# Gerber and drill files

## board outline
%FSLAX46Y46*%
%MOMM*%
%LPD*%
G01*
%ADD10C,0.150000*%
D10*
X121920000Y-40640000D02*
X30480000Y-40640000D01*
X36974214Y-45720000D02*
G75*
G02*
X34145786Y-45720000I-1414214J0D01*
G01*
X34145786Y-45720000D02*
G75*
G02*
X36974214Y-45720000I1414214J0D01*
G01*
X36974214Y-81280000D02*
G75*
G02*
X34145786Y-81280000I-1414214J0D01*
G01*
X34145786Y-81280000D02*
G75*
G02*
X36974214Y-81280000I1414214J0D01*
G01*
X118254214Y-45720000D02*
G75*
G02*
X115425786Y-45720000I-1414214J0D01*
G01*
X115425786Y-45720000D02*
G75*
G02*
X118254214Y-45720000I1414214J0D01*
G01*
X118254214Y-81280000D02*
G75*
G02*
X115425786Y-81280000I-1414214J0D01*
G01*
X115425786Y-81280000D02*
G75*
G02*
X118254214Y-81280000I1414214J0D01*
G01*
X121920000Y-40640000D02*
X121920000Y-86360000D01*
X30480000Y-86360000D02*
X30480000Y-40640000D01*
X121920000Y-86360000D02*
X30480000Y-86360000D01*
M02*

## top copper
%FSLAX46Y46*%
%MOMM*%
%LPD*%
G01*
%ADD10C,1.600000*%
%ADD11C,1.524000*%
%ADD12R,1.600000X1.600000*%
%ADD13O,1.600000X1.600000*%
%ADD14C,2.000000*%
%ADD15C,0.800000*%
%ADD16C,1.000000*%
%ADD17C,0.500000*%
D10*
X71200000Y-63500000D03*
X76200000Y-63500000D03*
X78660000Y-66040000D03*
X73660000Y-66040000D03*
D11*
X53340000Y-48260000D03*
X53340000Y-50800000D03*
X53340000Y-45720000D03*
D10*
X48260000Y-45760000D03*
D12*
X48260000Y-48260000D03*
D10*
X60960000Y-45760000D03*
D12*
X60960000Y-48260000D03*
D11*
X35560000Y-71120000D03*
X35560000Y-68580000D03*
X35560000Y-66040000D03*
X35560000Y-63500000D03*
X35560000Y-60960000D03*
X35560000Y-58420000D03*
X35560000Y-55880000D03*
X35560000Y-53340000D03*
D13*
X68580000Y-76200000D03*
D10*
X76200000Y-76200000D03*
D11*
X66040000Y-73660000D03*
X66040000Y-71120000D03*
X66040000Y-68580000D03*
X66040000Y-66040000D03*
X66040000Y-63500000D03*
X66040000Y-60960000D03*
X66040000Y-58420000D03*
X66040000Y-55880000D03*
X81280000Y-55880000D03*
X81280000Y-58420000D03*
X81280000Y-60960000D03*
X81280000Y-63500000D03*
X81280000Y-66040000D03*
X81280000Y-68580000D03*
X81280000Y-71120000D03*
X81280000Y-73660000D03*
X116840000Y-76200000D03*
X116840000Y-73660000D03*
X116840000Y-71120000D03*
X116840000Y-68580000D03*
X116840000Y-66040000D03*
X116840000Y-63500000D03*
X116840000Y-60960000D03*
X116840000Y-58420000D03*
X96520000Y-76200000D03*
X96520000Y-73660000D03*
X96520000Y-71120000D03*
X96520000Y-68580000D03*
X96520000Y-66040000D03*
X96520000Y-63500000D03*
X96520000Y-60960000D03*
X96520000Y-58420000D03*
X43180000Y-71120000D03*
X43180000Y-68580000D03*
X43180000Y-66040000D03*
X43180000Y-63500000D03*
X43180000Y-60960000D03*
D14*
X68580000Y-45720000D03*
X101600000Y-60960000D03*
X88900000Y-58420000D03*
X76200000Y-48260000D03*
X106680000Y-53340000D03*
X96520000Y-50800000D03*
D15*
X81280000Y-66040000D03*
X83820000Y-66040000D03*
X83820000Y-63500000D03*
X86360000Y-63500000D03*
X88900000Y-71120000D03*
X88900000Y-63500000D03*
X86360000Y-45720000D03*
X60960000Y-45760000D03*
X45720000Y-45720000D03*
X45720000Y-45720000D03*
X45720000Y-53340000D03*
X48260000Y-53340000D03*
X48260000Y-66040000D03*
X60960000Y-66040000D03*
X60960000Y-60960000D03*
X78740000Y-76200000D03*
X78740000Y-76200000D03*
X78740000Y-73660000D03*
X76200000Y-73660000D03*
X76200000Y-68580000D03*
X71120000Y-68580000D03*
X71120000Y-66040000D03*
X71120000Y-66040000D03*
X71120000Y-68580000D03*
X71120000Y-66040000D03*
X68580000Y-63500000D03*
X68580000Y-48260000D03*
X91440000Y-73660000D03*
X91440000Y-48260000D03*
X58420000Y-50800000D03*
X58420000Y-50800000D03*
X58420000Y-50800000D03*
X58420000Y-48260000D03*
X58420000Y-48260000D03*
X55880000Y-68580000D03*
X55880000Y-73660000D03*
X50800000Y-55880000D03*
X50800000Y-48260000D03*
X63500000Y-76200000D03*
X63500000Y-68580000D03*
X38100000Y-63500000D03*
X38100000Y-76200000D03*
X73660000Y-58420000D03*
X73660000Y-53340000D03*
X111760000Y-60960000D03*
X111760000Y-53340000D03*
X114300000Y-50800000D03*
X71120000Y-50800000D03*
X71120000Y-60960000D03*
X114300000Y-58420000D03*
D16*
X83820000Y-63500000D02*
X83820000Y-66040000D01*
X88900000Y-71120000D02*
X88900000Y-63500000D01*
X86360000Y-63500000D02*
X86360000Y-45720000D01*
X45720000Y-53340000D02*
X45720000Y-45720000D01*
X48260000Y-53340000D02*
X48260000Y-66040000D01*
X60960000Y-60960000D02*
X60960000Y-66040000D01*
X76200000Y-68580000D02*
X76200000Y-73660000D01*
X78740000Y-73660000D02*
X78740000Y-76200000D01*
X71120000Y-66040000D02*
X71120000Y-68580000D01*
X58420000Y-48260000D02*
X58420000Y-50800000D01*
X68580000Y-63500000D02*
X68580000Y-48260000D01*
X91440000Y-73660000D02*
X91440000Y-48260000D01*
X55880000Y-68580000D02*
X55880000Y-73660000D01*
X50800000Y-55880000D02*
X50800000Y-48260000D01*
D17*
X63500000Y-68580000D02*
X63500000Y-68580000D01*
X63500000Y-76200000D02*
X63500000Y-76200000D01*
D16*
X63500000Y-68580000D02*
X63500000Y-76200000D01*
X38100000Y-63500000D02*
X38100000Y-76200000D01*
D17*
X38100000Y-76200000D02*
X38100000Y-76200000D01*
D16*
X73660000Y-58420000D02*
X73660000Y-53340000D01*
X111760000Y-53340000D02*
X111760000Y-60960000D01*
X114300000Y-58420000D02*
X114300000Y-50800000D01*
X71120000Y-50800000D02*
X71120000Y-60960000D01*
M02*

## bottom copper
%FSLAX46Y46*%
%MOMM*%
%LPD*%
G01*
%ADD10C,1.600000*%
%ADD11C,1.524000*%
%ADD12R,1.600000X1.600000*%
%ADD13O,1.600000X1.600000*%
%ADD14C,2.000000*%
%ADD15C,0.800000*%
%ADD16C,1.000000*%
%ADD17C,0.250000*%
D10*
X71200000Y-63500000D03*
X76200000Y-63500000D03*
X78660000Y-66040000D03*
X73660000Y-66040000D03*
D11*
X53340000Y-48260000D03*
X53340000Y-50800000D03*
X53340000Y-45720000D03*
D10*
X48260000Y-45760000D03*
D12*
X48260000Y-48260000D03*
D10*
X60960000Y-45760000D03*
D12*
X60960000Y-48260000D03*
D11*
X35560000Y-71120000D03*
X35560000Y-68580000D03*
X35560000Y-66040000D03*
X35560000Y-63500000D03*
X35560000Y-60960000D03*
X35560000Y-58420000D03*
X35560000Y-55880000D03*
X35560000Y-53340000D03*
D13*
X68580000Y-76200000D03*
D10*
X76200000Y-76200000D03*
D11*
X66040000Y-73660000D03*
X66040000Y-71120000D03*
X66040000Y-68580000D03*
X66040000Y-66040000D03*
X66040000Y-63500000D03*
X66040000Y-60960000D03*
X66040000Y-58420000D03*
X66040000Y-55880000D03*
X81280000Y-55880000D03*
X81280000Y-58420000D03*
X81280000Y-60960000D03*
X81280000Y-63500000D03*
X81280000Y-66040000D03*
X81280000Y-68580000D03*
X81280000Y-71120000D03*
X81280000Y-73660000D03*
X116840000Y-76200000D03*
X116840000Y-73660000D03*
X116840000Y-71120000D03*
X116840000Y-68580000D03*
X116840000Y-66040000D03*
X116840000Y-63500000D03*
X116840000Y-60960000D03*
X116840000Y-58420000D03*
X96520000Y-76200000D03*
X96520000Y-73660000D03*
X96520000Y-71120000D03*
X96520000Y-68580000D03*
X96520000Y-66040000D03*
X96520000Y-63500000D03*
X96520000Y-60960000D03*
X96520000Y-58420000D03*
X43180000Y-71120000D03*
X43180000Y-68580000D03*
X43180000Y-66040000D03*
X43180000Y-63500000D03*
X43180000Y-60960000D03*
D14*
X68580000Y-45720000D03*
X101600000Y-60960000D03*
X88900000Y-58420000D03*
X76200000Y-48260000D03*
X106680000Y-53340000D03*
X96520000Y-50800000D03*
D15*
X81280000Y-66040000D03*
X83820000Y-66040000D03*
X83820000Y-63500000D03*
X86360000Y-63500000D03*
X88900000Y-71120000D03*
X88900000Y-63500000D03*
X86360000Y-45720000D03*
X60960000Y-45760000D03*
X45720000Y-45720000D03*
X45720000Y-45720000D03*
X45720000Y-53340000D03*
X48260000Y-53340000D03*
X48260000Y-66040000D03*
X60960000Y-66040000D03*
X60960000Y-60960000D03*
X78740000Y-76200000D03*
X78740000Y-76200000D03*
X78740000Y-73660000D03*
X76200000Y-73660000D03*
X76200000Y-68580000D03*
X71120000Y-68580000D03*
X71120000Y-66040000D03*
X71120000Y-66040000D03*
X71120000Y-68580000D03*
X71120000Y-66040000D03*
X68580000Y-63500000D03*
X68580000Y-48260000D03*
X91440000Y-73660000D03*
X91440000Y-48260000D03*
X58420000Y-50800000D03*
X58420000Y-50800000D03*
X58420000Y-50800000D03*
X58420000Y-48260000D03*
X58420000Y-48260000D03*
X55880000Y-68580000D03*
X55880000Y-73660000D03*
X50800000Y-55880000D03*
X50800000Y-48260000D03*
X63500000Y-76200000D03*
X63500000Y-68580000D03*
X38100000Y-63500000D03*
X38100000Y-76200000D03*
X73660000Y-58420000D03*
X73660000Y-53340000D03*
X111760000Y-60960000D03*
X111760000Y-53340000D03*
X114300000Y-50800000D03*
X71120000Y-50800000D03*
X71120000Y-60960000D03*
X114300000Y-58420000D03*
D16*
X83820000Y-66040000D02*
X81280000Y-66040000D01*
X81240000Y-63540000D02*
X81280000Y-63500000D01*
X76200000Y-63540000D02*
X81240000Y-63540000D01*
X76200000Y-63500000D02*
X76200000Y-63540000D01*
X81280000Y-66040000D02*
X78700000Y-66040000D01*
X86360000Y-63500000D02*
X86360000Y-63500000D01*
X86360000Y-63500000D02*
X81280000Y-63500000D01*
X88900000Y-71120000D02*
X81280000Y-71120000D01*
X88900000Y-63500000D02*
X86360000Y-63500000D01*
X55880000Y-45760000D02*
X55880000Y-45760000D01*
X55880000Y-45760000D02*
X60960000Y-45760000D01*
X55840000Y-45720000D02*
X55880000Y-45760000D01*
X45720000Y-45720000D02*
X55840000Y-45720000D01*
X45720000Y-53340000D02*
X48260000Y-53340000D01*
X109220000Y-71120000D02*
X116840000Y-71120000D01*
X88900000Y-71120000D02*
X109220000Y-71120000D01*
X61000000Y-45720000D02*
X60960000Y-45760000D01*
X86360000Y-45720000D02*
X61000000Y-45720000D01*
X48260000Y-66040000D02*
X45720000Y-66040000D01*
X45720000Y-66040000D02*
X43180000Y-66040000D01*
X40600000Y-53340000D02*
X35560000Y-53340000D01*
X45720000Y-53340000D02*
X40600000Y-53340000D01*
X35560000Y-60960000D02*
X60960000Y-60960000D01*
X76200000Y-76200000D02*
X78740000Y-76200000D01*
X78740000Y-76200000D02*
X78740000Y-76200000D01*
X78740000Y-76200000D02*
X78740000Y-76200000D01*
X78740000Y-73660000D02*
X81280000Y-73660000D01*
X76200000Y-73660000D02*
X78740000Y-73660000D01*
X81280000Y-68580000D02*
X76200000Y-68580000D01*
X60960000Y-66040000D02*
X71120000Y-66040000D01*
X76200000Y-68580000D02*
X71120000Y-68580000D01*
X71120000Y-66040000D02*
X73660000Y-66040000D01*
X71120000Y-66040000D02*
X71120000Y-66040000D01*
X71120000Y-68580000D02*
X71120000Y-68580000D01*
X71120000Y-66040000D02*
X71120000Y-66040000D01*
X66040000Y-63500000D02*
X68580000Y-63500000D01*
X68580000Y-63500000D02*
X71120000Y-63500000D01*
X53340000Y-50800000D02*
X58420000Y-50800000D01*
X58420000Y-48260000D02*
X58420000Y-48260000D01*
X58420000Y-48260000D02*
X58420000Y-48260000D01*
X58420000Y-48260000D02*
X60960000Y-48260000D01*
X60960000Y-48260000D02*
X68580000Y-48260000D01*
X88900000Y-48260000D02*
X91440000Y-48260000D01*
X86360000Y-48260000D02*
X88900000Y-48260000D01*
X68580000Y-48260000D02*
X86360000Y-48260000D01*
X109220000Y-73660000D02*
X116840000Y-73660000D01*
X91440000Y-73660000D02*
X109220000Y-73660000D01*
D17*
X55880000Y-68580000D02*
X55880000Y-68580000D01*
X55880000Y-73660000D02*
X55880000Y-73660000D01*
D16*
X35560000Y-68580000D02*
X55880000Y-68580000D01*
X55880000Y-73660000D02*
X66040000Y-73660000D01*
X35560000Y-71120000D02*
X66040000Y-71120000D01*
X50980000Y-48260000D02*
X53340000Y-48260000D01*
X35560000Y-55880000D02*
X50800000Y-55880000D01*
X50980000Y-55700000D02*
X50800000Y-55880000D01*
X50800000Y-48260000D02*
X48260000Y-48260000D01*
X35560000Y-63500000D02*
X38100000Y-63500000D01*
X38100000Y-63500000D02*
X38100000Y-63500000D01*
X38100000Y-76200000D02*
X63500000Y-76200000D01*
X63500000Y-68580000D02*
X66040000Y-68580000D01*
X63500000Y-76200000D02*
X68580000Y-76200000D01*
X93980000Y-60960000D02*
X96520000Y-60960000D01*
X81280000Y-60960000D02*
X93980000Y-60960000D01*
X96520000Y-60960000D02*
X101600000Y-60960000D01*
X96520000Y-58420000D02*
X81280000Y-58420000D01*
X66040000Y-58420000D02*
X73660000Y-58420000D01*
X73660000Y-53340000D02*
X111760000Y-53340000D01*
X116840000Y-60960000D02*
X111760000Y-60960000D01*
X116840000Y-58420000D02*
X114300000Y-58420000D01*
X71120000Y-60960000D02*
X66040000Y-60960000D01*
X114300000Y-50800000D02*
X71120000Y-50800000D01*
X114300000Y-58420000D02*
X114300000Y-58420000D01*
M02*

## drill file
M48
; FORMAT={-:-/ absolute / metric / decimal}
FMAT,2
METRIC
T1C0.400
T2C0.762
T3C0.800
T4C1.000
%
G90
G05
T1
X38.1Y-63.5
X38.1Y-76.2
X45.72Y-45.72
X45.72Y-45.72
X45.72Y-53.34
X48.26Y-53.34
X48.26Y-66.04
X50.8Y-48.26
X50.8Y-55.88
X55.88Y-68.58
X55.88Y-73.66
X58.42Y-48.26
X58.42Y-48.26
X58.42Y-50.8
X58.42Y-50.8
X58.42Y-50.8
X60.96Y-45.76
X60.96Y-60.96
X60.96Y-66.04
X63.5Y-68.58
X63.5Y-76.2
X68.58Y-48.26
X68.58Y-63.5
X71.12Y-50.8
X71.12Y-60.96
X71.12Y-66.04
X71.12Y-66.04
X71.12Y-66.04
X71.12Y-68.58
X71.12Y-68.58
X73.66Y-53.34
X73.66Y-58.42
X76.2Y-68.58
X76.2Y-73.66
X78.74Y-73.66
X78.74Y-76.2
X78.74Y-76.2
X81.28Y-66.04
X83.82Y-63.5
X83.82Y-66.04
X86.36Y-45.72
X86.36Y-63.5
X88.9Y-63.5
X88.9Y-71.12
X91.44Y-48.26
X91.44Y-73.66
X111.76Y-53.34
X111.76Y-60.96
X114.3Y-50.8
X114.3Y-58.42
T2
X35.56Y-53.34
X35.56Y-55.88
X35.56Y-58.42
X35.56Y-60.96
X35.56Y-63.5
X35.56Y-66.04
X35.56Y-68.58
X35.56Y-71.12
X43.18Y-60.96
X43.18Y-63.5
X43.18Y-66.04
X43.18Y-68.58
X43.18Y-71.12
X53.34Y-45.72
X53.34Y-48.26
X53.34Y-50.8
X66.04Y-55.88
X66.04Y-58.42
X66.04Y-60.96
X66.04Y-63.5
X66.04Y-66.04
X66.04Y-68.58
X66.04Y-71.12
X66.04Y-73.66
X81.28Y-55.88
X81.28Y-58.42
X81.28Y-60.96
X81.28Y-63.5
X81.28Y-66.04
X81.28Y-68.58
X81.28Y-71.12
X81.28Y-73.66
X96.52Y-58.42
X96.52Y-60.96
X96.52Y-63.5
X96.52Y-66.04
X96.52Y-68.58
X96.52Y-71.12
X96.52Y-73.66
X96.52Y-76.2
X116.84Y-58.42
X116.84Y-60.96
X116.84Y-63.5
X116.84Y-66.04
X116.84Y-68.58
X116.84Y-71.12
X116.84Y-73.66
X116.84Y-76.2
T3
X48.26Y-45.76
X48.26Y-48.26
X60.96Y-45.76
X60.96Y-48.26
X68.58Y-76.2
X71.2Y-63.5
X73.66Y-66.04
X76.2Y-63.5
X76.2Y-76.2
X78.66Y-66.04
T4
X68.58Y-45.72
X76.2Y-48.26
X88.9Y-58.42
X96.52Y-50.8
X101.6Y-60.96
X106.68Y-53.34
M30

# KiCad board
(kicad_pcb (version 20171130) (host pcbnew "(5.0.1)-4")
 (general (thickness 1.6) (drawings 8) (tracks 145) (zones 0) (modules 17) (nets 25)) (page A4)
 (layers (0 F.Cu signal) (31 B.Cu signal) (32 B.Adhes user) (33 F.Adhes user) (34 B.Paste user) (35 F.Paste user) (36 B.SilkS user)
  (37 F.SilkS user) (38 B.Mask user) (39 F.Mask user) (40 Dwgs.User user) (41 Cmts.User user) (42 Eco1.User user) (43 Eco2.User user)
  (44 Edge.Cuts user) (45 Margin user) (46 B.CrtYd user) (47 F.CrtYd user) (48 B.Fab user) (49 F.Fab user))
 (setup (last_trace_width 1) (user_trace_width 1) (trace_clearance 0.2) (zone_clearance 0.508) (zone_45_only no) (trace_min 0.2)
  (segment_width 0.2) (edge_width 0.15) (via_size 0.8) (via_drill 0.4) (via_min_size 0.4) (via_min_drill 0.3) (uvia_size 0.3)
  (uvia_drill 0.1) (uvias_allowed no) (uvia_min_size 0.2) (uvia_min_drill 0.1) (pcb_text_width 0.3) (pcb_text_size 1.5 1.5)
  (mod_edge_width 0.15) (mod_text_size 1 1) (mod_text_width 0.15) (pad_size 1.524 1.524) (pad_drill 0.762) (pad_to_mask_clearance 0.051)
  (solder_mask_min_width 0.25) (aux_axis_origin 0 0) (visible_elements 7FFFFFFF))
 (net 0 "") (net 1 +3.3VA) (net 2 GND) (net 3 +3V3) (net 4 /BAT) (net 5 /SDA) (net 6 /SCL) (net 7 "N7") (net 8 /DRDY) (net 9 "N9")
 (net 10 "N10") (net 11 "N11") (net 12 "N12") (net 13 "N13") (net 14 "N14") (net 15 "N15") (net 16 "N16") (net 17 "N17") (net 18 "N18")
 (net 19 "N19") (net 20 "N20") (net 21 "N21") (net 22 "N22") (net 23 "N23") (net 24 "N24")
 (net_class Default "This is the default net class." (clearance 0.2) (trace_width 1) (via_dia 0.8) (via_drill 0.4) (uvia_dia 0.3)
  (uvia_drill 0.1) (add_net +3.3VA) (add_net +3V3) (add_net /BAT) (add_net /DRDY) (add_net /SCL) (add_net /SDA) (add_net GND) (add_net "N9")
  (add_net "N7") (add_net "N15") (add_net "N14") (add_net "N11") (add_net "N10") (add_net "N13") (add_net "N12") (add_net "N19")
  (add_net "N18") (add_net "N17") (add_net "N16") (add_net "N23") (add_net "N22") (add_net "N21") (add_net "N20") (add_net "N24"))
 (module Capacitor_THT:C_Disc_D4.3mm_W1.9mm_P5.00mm (layer F.Cu) (at 76.2 63.5 180)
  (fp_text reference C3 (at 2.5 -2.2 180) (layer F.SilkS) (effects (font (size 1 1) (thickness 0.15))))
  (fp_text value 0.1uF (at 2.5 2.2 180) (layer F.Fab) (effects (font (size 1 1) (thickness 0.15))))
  (pad 2 thru_hole circle (at 5 0 180) (size 1.6 1.6) (drill 0.8) (layers *.Cu *.Mask) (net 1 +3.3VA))
  (pad 1 thru_hole circle (at 0 0 180) (size 1.6 1.6) (drill 0.8) (layers *.Cu *.Mask) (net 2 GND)))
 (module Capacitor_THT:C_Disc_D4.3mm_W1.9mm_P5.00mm (layer F.Cu) (at 73.66 66.04)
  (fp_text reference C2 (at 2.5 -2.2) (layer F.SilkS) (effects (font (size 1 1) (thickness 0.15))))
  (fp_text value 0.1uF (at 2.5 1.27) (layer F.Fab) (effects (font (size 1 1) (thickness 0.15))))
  (pad 2 thru_hole circle (at 5 0) (size 1.6 1.6) (drill 0.8) (layers *.Cu *.Mask) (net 2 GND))
  (pad 1 thru_hole circle (at 0 0) (size 1.6 1.6) (drill 0.8) (layers *.Cu *.Mask) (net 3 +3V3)))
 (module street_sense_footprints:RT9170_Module (layer F.Cu) (at 55.88 48.26 270)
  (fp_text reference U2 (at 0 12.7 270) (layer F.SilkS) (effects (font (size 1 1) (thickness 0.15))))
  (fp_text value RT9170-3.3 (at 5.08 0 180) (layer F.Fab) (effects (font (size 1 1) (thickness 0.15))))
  (pad 3 thru_hole circle (at 0 2.54 270) (size 1.524 1.524) (drill 0.762) (layers *.Cu *.Mask) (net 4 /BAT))
  (pad 2 thru_hole circle (at 2.54 2.54 270) (size 1.524 1.524) (drill 0.762) (layers *.Cu *.Mask) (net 1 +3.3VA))
  (pad 1 thru_hole circle (at -2.54 2.54 270) (size 1.524 1.524) (drill 0.762) (layers *.Cu *.Mask) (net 2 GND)))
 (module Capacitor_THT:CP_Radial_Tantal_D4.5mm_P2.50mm (layer F.Cu) (at 48.26 48.26 90)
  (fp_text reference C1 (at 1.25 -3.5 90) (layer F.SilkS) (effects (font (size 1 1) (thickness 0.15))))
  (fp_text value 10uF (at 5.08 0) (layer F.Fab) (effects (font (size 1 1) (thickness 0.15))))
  (pad 2 thru_hole circle (at 2.5 0 90) (size 1.6 1.6) (drill 0.8) (layers *.Cu *.Mask) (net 2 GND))
  (pad 1 thru_hole rect (at 0 0 90) (size 1.6 1.6) (drill 0.8) (layers *.Cu *.Mask) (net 4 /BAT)))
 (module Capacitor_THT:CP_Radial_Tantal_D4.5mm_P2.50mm (layer F.Cu) (at 60.96 48.26 90)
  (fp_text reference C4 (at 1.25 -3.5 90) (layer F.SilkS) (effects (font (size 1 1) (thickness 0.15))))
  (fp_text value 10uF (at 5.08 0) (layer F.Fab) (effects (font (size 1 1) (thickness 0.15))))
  (pad 2 thru_hole circle (at 2.5 0 90) (size 1.6 1.6) (drill 0.8) (layers *.Cu *.Mask) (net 2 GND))
  (pad 1 thru_hole rect (at 0 0 90) (size 1.6 1.6) (drill 0.8) (layers *.Cu *.Mask) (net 1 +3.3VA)))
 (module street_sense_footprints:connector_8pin (layer F.Cu) (at 35.56 50.8)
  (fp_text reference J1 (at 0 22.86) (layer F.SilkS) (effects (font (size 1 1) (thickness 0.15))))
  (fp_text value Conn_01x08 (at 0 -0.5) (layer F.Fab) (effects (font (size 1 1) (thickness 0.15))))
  (pad 8 thru_hole circle (at 0 20.32) (size 1.524 1.524) (drill 0.762) (layers *.Cu *.Mask) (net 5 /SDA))
  (pad 7 thru_hole circle (at 0 17.78) (size 1.524 1.524) (drill 0.762) (layers *.Cu *.Mask) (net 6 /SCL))
  (pad 6 thru_hole circle (at 0 15.24) (size 1.524 1.524) (drill 0.762) (layers *.Cu *.Mask) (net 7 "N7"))
  (pad 5 thru_hole circle (at 0 12.7) (size 1.524 1.524) (drill 0.762) (layers *.Cu *.Mask) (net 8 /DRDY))
  (pad 4 thru_hole circle (at 0 10.16) (size 1.524 1.524) (drill 0.762) (layers *.Cu *.Mask) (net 3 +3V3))
  (pad 3 thru_hole circle (at 0 7.62) (size 1.524 1.524) (drill 0.762) (layers *.Cu *.Mask) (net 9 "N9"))
  (pad 2 thru_hole circle (at 0 5.08) (size 1.524 1.524) (drill 0.762) (layers *.Cu *.Mask) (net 4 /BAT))
  (pad 1 thru_hole circle (at 0 2.54) (size 1.524 1.524) (drill 0.762) (layers *.Cu *.Mask) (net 2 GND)))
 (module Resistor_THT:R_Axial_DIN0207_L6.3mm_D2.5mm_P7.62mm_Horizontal (layer F.Cu) (at 76.2 76.2 180)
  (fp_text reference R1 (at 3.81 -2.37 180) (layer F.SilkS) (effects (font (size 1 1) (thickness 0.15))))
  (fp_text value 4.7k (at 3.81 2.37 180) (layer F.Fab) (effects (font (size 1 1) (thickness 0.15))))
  (pad 2 thru_hole oval (at 7.62 0 180) (size 1.6 1.6) (drill 0.8) (layers *.Cu *.Mask) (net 8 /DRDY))
  (pad 1 thru_hole circle (at 0 0 180) (size 1.6 1.6) (drill 0.8) (layers *.Cu *.Mask) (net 3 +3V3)))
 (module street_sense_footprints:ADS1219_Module (layer F.Cu) (at 76.2 76.2 180)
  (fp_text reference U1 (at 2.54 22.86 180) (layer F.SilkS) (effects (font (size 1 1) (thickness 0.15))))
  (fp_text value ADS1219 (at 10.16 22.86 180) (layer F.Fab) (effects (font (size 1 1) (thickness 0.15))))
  (pad 16 thru_hole circle (at 10.16 2.54 180) (size 1.524 1.524) (drill 0.762) (layers *.Cu *.Mask) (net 6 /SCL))
  (pad 15 thru_hole circle (at 10.16 5.08 180) (size 1.524 1.524) (drill 0.762) (layers *.Cu *.Mask) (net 5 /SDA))
  (pad 14 thru_hole circle (at 10.16 7.62 180) (size 1.524 1.524) (drill 0.762) (layers *.Cu *.Mask) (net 8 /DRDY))
  (pad 13 thru_hole circle (at 10.16 10.16 180) (size 1.524 1.524) (drill 0.762) (layers *.Cu *.Mask) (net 3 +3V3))
  (pad 12 thru_hole circle (at 10.16 12.7 180) (size 1.524 1.524) (drill 0.762) (layers *.Cu *.Mask) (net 1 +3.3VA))
  (pad 11 thru_hole circle (at 10.16 15.24 180) (size 1.524 1.524) (drill 0.762) (layers *.Cu *.Mask) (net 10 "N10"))
  (pad 10 thru_hole circle (at 10.16 17.78 180) (size 1.524 1.524) (drill 0.762) (layers *.Cu *.Mask) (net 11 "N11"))
  (pad 9 thru_hole circle (at 10.16 20.32 180) (size 1.524 1.524) (drill 0.762) (layers *.Cu *.Mask) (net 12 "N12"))
  (pad 8 thru_hole circle (at -5.08 20.32 180) (size 1.524 1.524) (drill 0.762) (layers *.Cu *.Mask) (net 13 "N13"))
  (pad 7 thru_hole circle (at -5.08 17.78 180) (size 1.524 1.524) (drill 0.762) (layers *.Cu *.Mask) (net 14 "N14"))
  (pad 6 thru_hole circle (at -5.08 15.24 180) (size 1.524 1.524) (drill 0.762) (layers *.Cu *.Mask) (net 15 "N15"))
  (pad 5 thru_hole circle (at -5.08 12.7 180) (size 1.524 1.524) (drill 0.762) (layers *.Cu *.Mask) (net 2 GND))
  (pad 4 thru_hole circle (at -5.08 10.16 180) (size 1.524 1.524) (drill 0.762) (layers *.Cu *.Mask) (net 2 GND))
  (pad 3 thru_hole circle (at -5.08 7.62 180) (size 1.524 1.524) (drill 0.762) (layers *.Cu *.Mask) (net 3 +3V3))
  (pad 2 thru_hole circle (at -5.08 5.08 180) (size 1.524 1.524) (drill 0.762) (layers *.Cu *.Mask) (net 2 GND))
  (pad 1 thru_hole circle (at -5.08 2.54 180) (size 1.524 1.524) (drill 0.762) (layers *.Cu *.Mask) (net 3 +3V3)))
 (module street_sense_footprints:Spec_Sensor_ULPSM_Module (layer F.Cu) (at 119.38 68.58 270)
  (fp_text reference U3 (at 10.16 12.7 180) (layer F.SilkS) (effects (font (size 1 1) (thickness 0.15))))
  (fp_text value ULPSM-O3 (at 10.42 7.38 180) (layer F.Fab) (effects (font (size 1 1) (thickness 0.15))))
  (pad 8 thru_hole circle (at 7.62 2.54 270) (size 1.524 1.524) (drill 0.762) (layers *.Cu *.Mask) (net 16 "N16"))
  (pad 7 thru_hole circle (at 5.08 2.54 270) (size 1.524 1.524) (drill 0.762) (layers *.Cu *.Mask) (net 1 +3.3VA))
  (pad 6 thru_hole circle (at 2.54 2.54 270) (size 1.524 1.524) (drill 0.762) (layers *.Cu *.Mask) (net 2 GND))
  (pad 5 thru_hole circle (at 0 2.54 270) (size 1.524 1.524) (drill 0.762) (layers *.Cu *.Mask) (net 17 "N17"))
  (pad 4 thru_hole circle (at -2.54 2.54 270) (size 1.524 1.524) (drill 0.762) (layers *.Cu *.Mask) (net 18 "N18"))
  (pad 3 thru_hole circle (at -5.08 2.54 270) (size 1.524 1.524) (drill 0.762) (layers *.Cu *.Mask) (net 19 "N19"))
  (pad 2 thru_hole circle (at -7.62 2.54 270) (size 1.524 1.524) (drill 0.762) (layers *.Cu *.Mask) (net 11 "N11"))
  (pad 1 thru_hole circle (at -10.16 2.54 270) (size 1.524 1.524) (drill 0.762) (layers *.Cu *.Mask) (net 10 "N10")))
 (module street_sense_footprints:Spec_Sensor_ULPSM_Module (layer F.Cu) (at 99.06 68.58 270)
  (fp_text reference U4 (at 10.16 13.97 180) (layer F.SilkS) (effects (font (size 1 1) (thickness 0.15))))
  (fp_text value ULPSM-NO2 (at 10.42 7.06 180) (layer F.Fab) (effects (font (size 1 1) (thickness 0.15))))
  (pad 8 thru_hole circle (at 7.62 2.54 270) (size 1.524 1.524) (drill 0.762) (layers *.Cu *.Mask) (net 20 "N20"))
  (pad 7 thru_hole circle (at 5.08 2.54 270) (size 1.524 1.524) (drill 0.762) (layers *.Cu *.Mask) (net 1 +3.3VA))
  (pad 6 thru_hole circle (at 2.54 2.54 270) (size 1.524 1.524) (drill 0.762) (layers *.Cu *.Mask) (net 2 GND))
  (pad 5 thru_hole circle (at 0 2.54 270) (size 1.524 1.524) (drill 0.762) (layers *.Cu *.Mask) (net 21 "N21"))
  (pad 4 thru_hole circle (at -2.54 2.54 270) (size 1.524 1.524) (drill 0.762) (layers *.Cu *.Mask) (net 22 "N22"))
  (pad 3 thru_hole circle (at -5.08 2.54 270) (size 1.524 1.524) (drill 0.762) (layers *.Cu *.Mask) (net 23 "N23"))
  (pad 2 thru_hole circle (at -7.62 2.54 270) (size 1.524 1.524) (drill 0.762) (layers *.Cu *.Mask) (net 15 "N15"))
  (pad 1 thru_hole circle (at -10.16 2.54 270) (size 1.524 1.524) (drill 0.762) (layers *.Cu *.Mask) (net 14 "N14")))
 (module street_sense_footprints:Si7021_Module (layer F.Cu) (at 53.34 66.04 270)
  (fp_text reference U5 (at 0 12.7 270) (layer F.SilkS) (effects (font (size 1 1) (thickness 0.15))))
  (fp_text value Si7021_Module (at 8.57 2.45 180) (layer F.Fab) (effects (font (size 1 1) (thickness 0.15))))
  (pad 5 thru_hole circle (at 5.08 10.16 270) (size 1.524 1.524) (drill 0.762) (layers *.Cu *.Mask) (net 5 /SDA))
  (pad 4 thru_hole circle (at 2.54 10.16 270) (size 1.524 1.524) (drill 0.762) (layers *.Cu *.Mask) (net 6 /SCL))
  (pad 3 thru_hole circle (at 0 10.16 270) (size 1.524 1.524) (drill 0.762) (layers *.Cu *.Mask) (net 2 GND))
  (pad 2 thru_hole circle (at -2.54 10.16 270) (size 1.524 1.524) (drill 0.762) (layers *.Cu *.Mask) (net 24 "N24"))
  (pad 1 thru_hole circle (at -5.08 10.16 270) (size 1.524 1.524) (drill 0.762) (layers *.Cu *.Mask) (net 3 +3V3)))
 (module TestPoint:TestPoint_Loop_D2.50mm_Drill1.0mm (layer F.Cu) (at 68.58 45.72)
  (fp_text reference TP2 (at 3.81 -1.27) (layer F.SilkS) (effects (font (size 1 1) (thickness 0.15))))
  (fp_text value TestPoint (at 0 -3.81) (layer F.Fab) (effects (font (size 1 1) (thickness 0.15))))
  (pad 1 thru_hole circle (at 0 0) (size 2 2) (drill 1) (layers *.Cu *.Mask) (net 2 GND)))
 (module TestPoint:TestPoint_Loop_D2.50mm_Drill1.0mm (layer F.Cu) (at 101.6 60.96)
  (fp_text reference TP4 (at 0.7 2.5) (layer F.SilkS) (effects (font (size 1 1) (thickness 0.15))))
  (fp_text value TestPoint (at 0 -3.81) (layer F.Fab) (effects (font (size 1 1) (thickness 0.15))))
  (pad 1 thru_hole circle (at 0 0) (size 2 2) (drill 1) (layers *.Cu *.Mask) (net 15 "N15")))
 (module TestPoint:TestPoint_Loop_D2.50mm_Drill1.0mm (layer F.Cu) (at 88.9 58.42)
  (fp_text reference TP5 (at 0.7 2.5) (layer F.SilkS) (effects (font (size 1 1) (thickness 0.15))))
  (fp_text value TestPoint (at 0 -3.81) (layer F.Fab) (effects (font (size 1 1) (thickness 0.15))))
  (pad 1 thru_hole circle (at 0 0) (size 2 2) (drill 1) (layers *.Cu *.Mask) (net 14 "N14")))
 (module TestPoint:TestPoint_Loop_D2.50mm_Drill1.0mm (layer F.Cu) (at 76.2 48.26)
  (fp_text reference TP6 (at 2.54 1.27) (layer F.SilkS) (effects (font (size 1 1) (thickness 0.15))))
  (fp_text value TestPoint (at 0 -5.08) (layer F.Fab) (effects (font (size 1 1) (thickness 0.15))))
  (pad 1 thru_hole circle (at 0 0) (size 2 2) (drill 1) (layers *.Cu *.Mask) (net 1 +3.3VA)))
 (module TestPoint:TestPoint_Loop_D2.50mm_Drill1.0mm (layer F.Cu) (at 106.68 53.34)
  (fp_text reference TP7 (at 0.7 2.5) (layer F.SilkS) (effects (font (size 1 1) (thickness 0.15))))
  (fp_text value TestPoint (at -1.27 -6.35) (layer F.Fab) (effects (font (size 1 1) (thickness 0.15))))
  (pad 1 thru_hole circle (at 0 0) (size 2 2) (drill 1) (layers *.Cu *.Mask) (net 11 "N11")))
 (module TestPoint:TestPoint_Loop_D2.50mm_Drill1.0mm (layer F.Cu) (at 96.52 50.8)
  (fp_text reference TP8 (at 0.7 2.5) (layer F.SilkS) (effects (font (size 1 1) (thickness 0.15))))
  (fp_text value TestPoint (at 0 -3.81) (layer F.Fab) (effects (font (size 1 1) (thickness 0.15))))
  (pad 1 thru_hole circle (at 0 0) (size 2 2) (drill 1) (layers *.Cu *.Mask) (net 10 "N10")))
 (gr_line (start 121.92 40.64) (end 30.48 40.64) (layer Edge.Cuts) (width 0.15))
 (gr_circle (center 35.56 45.72) (end 36.974214 45.72) (layer Edge.Cuts) (width 0.15))
 (gr_circle (center 35.56 81.28) (end 36.974214 81.28) (layer Edge.Cuts) (width 0.15))
 (gr_circle (center 116.84 45.72) (end 115.84 46.72) (layer Edge.Cuts) (width 0.15))
 (gr_circle (center 116.84 81.28) (end 118.254214 81.28) (layer Edge.Cuts) (width 0.15))
 (gr_line (start 121.92 40.64) (end 121.92 86.36) (layer Edge.Cuts) (width 0.15))
 (gr_line (start 30.48 86.36) (end 30.48 40.64) (layer Edge.Cuts) (width 0.15))
 (gr_line (start 121.92 86.36) (end 30.48 86.36) (layer Edge.Cuts) (width 0.15))
 (via (at 81.28 66.04) (size 0.8) (drill 0.4) (layers F.Cu B.Cu) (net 2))
 (via (at 83.82 66.04) (size 0.8) (drill 0.4) (layers F.Cu B.Cu) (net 2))
 (segment (start 83.82 66.04) (end 81.28 66.04) (width 1) (layer B.Cu) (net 2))
 (segment (start 81.24 63.54) (end 81.28 63.5) (width 1) (layer B.Cu) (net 2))
 (segment (start 76.2 63.54) (end 81.24 63.54) (width 1) (layer B.Cu) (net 2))
 (segment (start 76.2 63.5) (end 76.2 63.54) (width 1) (layer B.Cu) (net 2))
 (segment (start 83.82 63.5) (end 83.82 66.04) (width 1) (layer F.Cu) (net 2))
 (via (at 83.82 63.5) (size 0.8) (drill 0.4) (layers F.Cu B.Cu) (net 2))
 (segment (start 81.28 66.04) (end 78.7 66.04) (width 1) (layer B.Cu) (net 2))
 (segment (start 86.36 63.5) (end 86.36 63.5) (width 1) (layer B.Cu) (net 2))
 (segment (start 86.36 63.5) (end 81.28 63.5) (width 1) (layer B.Cu) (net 2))
 (via (at 86.36 63.5) (size 0.8) (drill 0.4) (layers F.Cu B.Cu) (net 2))
 (via (at 88.9 71.12) (size 0.8) (drill 0.4) (layers F.Cu B.Cu) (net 2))
 (segment (start 88.9 71.12) (end 81.28 71.12) (width 1) (layer B.Cu) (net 2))
 (via (at 88.9 63.5) (size 0.8) (drill 0.4) (layers F.Cu B.Cu) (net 2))
 (segment (start 88.9 71.12) (end 88.9 63.5) (width 1) (layer F.Cu) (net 2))
 (segment (start 88.9 63.5) (end 86.36 63.5) (width 1) (layer B.Cu) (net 2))
 (via (at 86.36 45.72) (size 0.8) (drill 0.4) (layers F.Cu B.Cu) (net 2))
 (segment (start 55.88 45.76) (end 55.88 45.76) (width 1) (layer B.Cu) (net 2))
 (via (at 60.96 45.76) (size 0.8) (drill 0.4) (layers F.Cu B.Cu) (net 2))
 (segment (start 55.88 45.76) (end 60.96 45.76) (width 1) (layer B.Cu) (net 2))
 (segment (start 86.36 63.5) (end 86.36 45.72) (width 1) (layer F.Cu) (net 2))
 (segment (start 45.72 53.34) (end 45.72 45.72) (width 1) (layer F.Cu) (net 2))
 (segment (start 55.84 45.72) (end 55.88 45.76) (width 1) (layer B.Cu) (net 2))
 (segment (start 45.72 45.72) (end 55.84 45.72) (width 1) (layer B.Cu) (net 2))
 (via (at 45.72 45.72) (size 0.8) (drill 0.4) (layers F.Cu B.Cu) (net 2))
 (via (at 45.72 45.72) (size 0.8) (drill 0.4) (layers F.Cu B.Cu) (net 2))
 (via (at 45.72 53.34) (size 0.8) (drill 0.4) (layers F.Cu B.Cu) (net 2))
 (segment (start 45.72 53.34) (end 48.26 53.34) (width 1) (layer B.Cu) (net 2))
 (via (at 48.26 53.34) (size 0.8) (drill 0.4) (layers F.Cu B.Cu) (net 2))
 (segment (start 109.22 71.12) (end 116.84 71.12) (width 1) (layer B.Cu) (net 2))
 (segment (start 88.9 71.12) (end 109.22 71.12) (width 1) (layer B.Cu) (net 2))
 (segment (start 61 45.72) (end 60.96 45.76) (width 1) (layer B.Cu) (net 2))
 (segment (start 86.36 45.72) (end 61 45.72) (width 1) (layer B.Cu) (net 2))
 (segment (start 48.26 53.34) (end 48.26 66.04) (width 1) (layer F.Cu) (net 2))
 (segment (start 48.26 66.04) (end 45.72 66.04) (width 1) (layer B.Cu) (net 2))
 (segment (start 45.72 66.04) (end 43.18 66.04) (width 1) (layer B.Cu) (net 2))
 (via (at 48.26 66.04) (size 0.8) (drill 0.4) (layers F.Cu B.Cu) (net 2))
 (segment (start 40.6 53.34) (end 35.56 53.34) (width 1) (layer B.Cu) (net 2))
 (segment (start 45.72 53.34) (end 40.6 53.34) (width 1) (layer B.Cu) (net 2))
 (via (at 60.96 66.04) (size 0.8) (drill 0.4) (layers F.Cu B.Cu) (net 3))
 (segment (start 35.56 60.96) (end 60.96 60.96) (width 1) (layer B.Cu) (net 3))
 (segment (start 60.96 60.96) (end 60.96 66.04) (width 1) (layer F.Cu) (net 3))
 (via (at 60.96 60.96) (size 0.8) (drill 0.4) (layers F.Cu B.Cu) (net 3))
 (segment (start 76.2 68.58) (end 76.2 73.66) (width 1) (layer F.Cu) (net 3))
 (segment (start 76.2 76.2) (end 78.74 76.2) (width 1) (layer B.Cu) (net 3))
 (segment (start 78.74 76.2) (end 78.74 76.2) (width 1) (layer B.Cu) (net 3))
 (via (at 78.74 76.2) (size 0.8) (drill 0.4) (layers F.Cu B.Cu) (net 3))
 (segment (start 78.74 76.2) (end 78.74 76.2) (width 1) (layer B.Cu) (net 3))
 (via (at 78.74 76.2) (size 0.8) (drill 0.4) (layers F.Cu B.Cu) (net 3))
 (segment (start 78.74 73.66) (end 81.28 73.66) (width 1) (layer B.Cu) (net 3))
 (via (at 78.74 73.66) (size 0.8) (drill 0.4) (layers F.Cu B.Cu) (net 3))
 (segment (start 78.74 73.66) (end 78.74 76.2) (width 1) (layer F.Cu) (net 3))
 (segment (start 76.2 73.66) (end 78.74 73.66) (width 1) (layer B.Cu) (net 3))
 (via (at 76.2 73.66) (size 0.8) (drill 0.4) (layers F.Cu B.Cu) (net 3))
 (via (at 76.2 68.58) (size 0.8) (drill 0.4) (layers F.Cu B.Cu) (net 3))
 (segment (start 81.28 68.58) (end 76.2 68.58) (width 1) (layer B.Cu) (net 3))
 (segment (start 60.96 66.04) (end 71.12 66.04) (width 1) (layer B.Cu) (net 3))
 (segment (start 76.2 68.58) (end 71.12 68.58) (width 1) (layer B.Cu) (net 3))
 (via (at 71.12 68.58) (size 0.8) (drill 0.4) (layers F.Cu B.Cu) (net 3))
 (segment (start 71.12 66.04) (end 73.66 66.04) (width 1) (layer B.Cu) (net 3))
 (via (at 71.12 66.04) (size 0.8) (drill 0.4) (layers F.Cu B.Cu) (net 3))
 (segment (start 71.12 66.04) (end 71.12 66.04) (width 1) (layer B.Cu) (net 3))
 (via (at 71.12 66.04) (size 0.8) (drill 0.4) (layers F.Cu B.Cu) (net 3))
 (segment (start 71.12 68.58) (end 71.12 68.58) (width 1) (layer B.Cu) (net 3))
 (via (at 71.12 68.58) (size 0.8) (drill 0.4) (layers F.Cu B.Cu) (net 3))
 (segment (start 71.12 66.04) (end 71.12 66.04) (width 1) (layer B.Cu) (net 3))
 (via (at 71.12 66.04) (size 0.8) (drill 0.4) (layers F.Cu B.Cu) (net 3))
 (segment (start 71.12 66.04) (end 71.12 68.58) (width 1) (layer F.Cu) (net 3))
 (via (at 68.58 63.5) (size 0.8) (drill 0.4) (layers F.Cu B.Cu) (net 1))
 (segment (start 66.04 63.5) (end 68.58 63.5) (width 1) (layer B.Cu) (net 1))
 (via (at 68.58 48.26) (size 0.8) (drill 0.4) (layers F.Cu B.Cu) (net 1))
 (via (at 91.44 73.66) (size 0.8) (drill 0.4) (layers F.Cu B.Cu) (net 1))
 (segment (start 68.58 63.5) (end 71.12 63.5) (width 1) (layer B.Cu) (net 1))
 (via (at 91.44 48.26) (size 0.8) (drill 0.4) (layers F.Cu B.Cu) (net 1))
 (segment (start 58.42 48.26) (end 58.42 50.8) (width 1) (layer F.Cu) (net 1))
 (via (at 58.42 50.8) (size 0.8) (drill 0.4) (layers F.Cu B.Cu) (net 1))
 (via (at 58.42 50.8) (size 0.8) (drill 0.4) (layers F.Cu B.Cu) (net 1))
 (via (at 58.42 50.8) (size 0.8) (drill 0.4) (layers F.Cu B.Cu) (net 1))
 (segment (start 53.34 50.8) (end 58.42 50.8) (width 1) (layer B.Cu) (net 1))
 (segment (start 58.42 48.26) (end 58.42 48.26) (width 1) (layer B.Cu) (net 1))
 (segment (start 58.42 48.26) (end 58.42 48.26) (width 1) (layer B.Cu) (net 1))
 (via (at 58.42 48.26) (size 0.8) (drill 0.4) (layers F.Cu B.Cu) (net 1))
 (via (at 58.42 48.26) (size 0.8) (drill 0.4) (layers F.Cu B.Cu) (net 1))
 (segment (start 58.42 48.26) (end 60.96 48.26) (width 1) (layer B.Cu) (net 1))
 (segment (start 60.96 48.26) (end 68.58 48.26) (width 1) (layer B.Cu) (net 1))
 (segment (start 88.9 48.26) (end 91.44 48.26) (width 1) (layer B.Cu) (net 1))
 (segment (start 86.36 48.26) (end 88.9 48.26) (width 1) (layer B.Cu) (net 1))
 (segment (start 68.58 48.26) (end 86.36 48.26) (width 1) (layer B.Cu) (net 1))
 (segment (start 68.58 63.5) (end 68.58 48.26) (width 1) (layer F.Cu) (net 1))
 (segment (start 91.44 73.66) (end 91.44 48.26) (width 1) (layer F.Cu) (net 1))
 (segment (start 109.22 73.66) (end 116.84 73.66) (width 1) (layer B.Cu) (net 1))
 (segment (start 91.44 73.66) (end 109.22 73.66) (width 1) (layer B.Cu) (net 1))
 (segment (start 55.88 68.58) (end 55.88 68.58) (width 0.25) (layer B.Cu) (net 6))
 (via (at 55.88 68.58) (size 0.8) (drill 0.4) (layers F.Cu B.Cu) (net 6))
 (segment (start 55.88 73.66) (end 55.88 73.66) (width 0.25) (layer B.Cu) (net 6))
 (via (at 55.88 73.66) (size 0.8) (drill 0.4) (layers F.Cu B.Cu) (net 6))
 (segment (start 35.56 68.58) (end 55.88 68.58) (width 1) (layer B.Cu) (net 6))
 (segment (start 55.88 73.66) (end 66.04 73.66) (width 1) (layer B.Cu) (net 6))
 (segment (start 55.88 68.58) (end 55.88 73.66) (width 1) (layer F.Cu) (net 6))
 (segment (start 35.56 71.12) (end 66.04 71.12) (width 1) (layer B.Cu) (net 5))
 (segment (start 50.98 48.26) (end 53.34 48.26) (width 1) (layer B.Cu) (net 4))
 (segment (start 35.56 55.88) (end 50.8 55.88) (width 1) (layer B.Cu) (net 4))
 (via (at 50.8 55.88) (size 0.8) (drill 0.4) (layers F.Cu B.Cu) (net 4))
 (segment (start 50.98 55.7) (end 50.8 55.88) (width 1) (layer B.Cu) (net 4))
 (segment (start 50.8 55.88) (end 50.8 48.26) (width 1) (layer F.Cu) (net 4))
 (via (at 50.8 48.26) (size 0.8) (drill 0.4) (layers F.Cu B.Cu) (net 4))
 (segment (start 50.8 48.26) (end 48.26 48.26) (width 1) (layer B.Cu) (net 4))
 (segment (start 63.5 68.58) (end 63.5 68.58) (width 0.5) (layer F.Cu) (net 8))
 (segment (start 63.5 76.2) (end 63.5 76.2) (width 0.5) (layer F.Cu) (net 8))
 (via (at 63.5 76.2) (size 0.8) (drill 0.4) (layers F.Cu B.Cu) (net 8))
 (segment (start 63.5 68.58) (end 63.5 76.2) (width 1) (layer F.Cu) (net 8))
 (via (at 63.5 68.58) (size 0.8) (drill 0.4) (layers F.Cu B.Cu) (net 8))
 (segment (start 35.56 63.5) (end 38.1 63.5) (width 1) (layer B.Cu) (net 8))
 (segment (start 38.1 63.5) (end 38.1 63.5) (width 1) (layer B.Cu) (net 8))
 (via (at 38.1 63.5) (size 0.8) (drill 0.4) (layers F.Cu B.Cu) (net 8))
 (segment (start 38.1 63.5) (end 38.1 76.2) (width 1) (layer F.Cu) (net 8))
 (segment (start 38.1 76.2) (end 38.1 76.2) (width 0.5) (layer F.Cu) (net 8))
 (via (at 38.1 76.2) (size 0.8) (drill 0.4) (layers F.Cu B.Cu) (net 8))
 (segment (start 38.1 76.2) (end 63.5 76.2) (width 1) (layer B.Cu) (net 8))
 (segment (start 63.5 68.58) (end 66.04 68.58) (width 1) (layer B.Cu) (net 8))
 (segment (start 63.5 76.2) (end 68.58 76.2) (width 1) (layer B.Cu) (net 8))
 (segment (start 93.98 60.96) (end 96.52 60.96) (width 1) (layer B.Cu) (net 15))
 (segment (start 81.28 60.96) (end 93.98 60.96) (width 1) (layer B.Cu) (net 15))
 (segment (start 96.52 60.96) (end 101.6 60.96) (width 1) (layer B.Cu) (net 15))
 (segment (start 96.52 58.42) (end 81.28 58.42) (width 1) (layer B.Cu) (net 14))
 (via (at 73.66 58.42) (size 0.8) (drill 0.4) (layers F.Cu B.Cu) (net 11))
 (segment (start 66.04 58.42) (end 73.66 58.42) (width 1) (layer B.Cu) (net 11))
 (via (at 73.66 53.34) (size 0.8) (drill 0.4) (layers F.Cu B.Cu) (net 11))
 (segment (start 73.66 58.42) (end 73.66 53.34) (width 1) (layer F.Cu) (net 11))
 (via (at 111.76 60.96) (size 0.8) (drill 0.4) (layers F.Cu B.Cu) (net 11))
 (via (at 111.76 53.34) (size 0.8) (drill 0.4) (layers F.Cu B.Cu) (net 11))
 (segment (start 111.76 53.34) (end 111.76 60.96) (width 1) (layer F.Cu) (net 11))
 (segment (start 73.66 53.34) (end 111.76 53.34) (width 1) (layer B.Cu) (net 11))
 (segment (start 116.84 60.96) (end 111.76 60.96) (width 1) (layer B.Cu) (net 11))
 (segment (start 116.84 58.42) (end 114.3 58.42) (width 1) (layer B.Cu) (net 10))
 (via (at 114.3 50.8) (size 0.8) (drill 0.4) (layers F.Cu B.Cu) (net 10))
 (segment (start 114.3 58.42) (end 114.3 50.8) (width 1) (layer F.Cu) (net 10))
 (via (at 71.12 50.8) (size 0.8) (drill 0.4) (layers F.Cu B.Cu) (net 10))
 (via (at 71.12 60.96) (size 0.8) (drill 0.4) (layers F.Cu B.Cu) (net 10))
 (segment (start 71.12 50.8) (end 71.12 60.96) (width 1) (layer F.Cu) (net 10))
 (segment (start 71.12 60.96) (end 66.04 60.96) (width 1) (layer B.Cu) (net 10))
 (segment (start 114.3 50.8) (end 71.12 50.8) (width 1) (layer B.Cu) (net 10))
 (segment (start 114.3 58.42) (end 114.3 58.42) (width 1) (layer B.Cu) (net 10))
 (via (at 114.3 58.42) (size 0.8) (drill 0.4) (layers F.Cu B.Cu) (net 10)))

